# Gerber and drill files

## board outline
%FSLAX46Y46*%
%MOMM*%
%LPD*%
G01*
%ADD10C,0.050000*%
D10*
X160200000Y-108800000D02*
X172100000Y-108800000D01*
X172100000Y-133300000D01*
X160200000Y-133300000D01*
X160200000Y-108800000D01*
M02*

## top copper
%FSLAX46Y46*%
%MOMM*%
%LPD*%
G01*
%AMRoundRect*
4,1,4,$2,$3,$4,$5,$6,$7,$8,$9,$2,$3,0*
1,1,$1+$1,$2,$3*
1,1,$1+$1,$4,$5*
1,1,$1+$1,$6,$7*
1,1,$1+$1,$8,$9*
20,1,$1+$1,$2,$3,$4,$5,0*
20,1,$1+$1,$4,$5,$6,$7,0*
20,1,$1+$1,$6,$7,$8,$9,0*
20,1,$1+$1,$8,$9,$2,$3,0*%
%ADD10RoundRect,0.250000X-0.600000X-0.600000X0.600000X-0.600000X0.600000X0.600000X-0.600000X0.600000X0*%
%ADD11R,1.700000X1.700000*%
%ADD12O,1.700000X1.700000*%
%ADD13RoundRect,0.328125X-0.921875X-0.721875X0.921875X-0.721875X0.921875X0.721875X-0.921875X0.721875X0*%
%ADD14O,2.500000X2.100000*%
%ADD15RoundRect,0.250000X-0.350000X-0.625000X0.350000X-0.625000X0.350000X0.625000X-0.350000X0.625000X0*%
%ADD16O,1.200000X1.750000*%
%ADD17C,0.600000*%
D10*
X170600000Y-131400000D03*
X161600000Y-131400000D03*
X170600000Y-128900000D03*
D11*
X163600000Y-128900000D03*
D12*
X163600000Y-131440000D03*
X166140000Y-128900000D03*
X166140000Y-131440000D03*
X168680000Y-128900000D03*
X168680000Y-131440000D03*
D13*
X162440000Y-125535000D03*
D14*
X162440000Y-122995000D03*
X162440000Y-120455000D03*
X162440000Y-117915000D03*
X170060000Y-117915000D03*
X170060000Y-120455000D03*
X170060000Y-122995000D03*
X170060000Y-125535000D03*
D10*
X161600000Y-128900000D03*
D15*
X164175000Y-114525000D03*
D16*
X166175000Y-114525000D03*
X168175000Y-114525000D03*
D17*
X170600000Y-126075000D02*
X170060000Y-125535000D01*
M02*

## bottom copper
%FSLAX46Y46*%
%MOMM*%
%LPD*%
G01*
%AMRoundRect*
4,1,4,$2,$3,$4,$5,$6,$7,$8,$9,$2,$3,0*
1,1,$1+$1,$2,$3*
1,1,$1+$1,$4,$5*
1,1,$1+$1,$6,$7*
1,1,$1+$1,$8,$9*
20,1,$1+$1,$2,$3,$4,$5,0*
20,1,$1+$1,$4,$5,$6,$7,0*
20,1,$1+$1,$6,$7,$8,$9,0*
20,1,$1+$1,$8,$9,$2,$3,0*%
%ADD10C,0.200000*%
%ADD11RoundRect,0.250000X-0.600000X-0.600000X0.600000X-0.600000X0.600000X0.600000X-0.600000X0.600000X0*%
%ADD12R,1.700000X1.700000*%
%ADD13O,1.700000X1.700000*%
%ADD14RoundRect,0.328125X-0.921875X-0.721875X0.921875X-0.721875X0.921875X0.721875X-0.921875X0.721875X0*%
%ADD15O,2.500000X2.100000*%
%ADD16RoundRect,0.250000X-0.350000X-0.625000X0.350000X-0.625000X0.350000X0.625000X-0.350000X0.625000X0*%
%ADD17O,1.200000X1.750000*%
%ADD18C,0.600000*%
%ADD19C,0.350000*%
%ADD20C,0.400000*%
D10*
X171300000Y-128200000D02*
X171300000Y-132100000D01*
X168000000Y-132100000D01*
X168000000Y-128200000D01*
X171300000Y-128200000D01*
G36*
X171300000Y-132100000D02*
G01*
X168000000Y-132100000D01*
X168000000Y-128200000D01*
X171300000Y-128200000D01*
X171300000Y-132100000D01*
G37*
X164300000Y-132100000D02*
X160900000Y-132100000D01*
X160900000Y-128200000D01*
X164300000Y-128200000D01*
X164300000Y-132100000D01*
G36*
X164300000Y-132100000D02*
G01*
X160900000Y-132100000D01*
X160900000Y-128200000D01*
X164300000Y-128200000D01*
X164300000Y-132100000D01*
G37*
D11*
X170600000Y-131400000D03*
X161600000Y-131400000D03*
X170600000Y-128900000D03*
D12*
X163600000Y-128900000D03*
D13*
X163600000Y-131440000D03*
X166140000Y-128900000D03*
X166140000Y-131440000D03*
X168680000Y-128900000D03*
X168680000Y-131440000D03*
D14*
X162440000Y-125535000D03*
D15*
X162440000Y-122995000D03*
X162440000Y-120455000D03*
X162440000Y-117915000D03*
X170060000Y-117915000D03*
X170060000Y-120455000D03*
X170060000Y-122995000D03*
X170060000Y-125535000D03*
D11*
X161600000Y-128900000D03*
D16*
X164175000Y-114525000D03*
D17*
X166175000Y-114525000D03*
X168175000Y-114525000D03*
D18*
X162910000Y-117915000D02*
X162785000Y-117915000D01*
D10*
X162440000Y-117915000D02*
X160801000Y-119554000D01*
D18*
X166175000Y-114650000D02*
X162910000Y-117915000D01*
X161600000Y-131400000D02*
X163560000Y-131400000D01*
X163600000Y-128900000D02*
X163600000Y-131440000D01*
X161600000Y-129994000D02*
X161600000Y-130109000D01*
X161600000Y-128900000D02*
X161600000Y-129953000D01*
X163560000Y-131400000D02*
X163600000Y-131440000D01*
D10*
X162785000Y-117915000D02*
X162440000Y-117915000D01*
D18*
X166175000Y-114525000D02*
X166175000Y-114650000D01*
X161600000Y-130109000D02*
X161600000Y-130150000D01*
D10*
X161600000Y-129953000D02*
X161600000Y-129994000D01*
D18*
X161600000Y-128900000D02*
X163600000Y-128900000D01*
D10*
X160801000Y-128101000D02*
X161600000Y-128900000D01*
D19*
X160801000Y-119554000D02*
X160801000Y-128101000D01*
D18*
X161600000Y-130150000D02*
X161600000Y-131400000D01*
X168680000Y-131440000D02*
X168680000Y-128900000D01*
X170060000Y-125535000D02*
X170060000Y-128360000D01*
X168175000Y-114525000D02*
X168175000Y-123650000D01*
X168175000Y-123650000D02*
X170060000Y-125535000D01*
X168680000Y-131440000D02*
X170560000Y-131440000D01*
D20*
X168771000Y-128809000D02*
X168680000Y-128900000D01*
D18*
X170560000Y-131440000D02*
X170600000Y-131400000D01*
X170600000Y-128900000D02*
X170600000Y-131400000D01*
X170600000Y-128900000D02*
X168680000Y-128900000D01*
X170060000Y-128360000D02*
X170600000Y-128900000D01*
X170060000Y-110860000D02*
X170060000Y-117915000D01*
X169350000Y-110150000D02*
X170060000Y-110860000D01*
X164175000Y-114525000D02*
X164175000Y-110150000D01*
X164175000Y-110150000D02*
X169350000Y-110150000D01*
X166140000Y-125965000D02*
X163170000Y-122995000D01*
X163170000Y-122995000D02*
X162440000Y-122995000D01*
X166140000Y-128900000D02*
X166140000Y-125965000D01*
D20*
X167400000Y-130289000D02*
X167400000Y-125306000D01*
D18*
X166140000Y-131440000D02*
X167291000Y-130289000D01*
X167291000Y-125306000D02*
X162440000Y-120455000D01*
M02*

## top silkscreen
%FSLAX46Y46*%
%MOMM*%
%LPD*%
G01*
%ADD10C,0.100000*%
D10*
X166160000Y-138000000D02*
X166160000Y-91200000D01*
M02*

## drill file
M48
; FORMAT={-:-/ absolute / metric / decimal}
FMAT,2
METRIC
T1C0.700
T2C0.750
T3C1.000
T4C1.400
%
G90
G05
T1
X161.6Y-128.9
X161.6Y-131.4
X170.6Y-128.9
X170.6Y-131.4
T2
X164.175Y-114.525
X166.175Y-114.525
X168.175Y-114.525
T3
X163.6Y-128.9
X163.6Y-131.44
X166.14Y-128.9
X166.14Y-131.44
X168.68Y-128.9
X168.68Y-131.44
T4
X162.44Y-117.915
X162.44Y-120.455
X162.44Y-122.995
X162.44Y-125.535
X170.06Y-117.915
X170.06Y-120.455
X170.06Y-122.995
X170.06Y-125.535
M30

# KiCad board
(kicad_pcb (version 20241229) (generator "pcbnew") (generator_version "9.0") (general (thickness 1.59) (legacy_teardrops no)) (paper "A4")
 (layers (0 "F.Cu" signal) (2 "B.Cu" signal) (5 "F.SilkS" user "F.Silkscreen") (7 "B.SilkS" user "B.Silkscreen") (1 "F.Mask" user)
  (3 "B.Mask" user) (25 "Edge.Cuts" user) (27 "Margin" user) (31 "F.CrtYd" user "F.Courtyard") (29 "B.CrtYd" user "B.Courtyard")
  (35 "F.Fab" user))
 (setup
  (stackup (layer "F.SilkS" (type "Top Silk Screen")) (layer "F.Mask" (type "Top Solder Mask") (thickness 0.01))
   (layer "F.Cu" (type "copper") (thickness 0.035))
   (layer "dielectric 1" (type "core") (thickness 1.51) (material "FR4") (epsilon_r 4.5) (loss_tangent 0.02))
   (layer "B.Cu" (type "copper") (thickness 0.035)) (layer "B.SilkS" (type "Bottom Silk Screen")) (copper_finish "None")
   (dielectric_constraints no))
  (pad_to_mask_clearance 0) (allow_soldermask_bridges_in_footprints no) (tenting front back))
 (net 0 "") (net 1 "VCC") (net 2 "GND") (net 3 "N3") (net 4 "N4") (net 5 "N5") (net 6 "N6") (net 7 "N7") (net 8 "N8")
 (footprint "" (layer "F.Cu") (at 170.6 131.4)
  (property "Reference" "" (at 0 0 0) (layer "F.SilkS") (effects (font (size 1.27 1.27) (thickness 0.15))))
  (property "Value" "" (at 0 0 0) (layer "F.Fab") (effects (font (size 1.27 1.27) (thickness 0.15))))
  (pad "1" thru_hole roundrect (at 0 0) (size 1.7 1.7) (drill 0.7) (layers "*.Cu" "*.Mask") (remove_unused_layers no)
   (roundrect_rratio 0.147059) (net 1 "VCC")))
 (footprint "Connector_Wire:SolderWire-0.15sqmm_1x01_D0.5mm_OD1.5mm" (layer "B.Cu") (at 161.6 131.4)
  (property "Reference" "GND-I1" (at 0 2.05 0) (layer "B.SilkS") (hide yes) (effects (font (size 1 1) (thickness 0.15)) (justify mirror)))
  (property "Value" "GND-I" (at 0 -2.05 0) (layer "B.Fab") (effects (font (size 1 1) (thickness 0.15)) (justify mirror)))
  (pad "1" thru_hole roundrect (at 0 0) (size 1.7 1.7) (drill 0.7) (layers "*.Cu" "*.Mask") (remove_unused_layers no)
   (roundrect_rratio 0.147059) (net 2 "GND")))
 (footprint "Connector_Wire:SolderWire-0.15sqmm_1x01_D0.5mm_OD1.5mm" (layer "B.Cu") (at 170.6 128.9)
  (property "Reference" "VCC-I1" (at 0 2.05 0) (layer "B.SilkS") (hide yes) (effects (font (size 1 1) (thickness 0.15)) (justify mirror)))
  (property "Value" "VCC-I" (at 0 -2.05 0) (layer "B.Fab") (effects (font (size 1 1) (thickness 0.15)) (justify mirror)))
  (pad "1" thru_hole roundrect (at 0 0) (size 1.7 1.7) (drill 0.7) (layers "*.Cu" "*.Mask") (remove_unused_layers no)
   (roundrect_rratio 0.147059) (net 1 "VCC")))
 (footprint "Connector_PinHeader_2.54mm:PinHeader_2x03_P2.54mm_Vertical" (layer "B.Cu") (at 163.6 128.9 -90)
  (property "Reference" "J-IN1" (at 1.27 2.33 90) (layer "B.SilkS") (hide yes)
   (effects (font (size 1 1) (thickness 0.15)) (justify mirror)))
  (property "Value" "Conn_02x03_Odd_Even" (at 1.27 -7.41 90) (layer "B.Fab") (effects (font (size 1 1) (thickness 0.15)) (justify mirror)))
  (pad "1" thru_hole rect (at 0 0 270) (size 1.7 1.7) (drill 1) (layers "*.Cu" "*.Mask") (remove_unused_layers no) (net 2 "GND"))
  (pad "2" thru_hole oval (at 2.54 0 270) (size 1.7 1.7) (drill 1) (layers "*.Cu" "*.Mask") (remove_unused_layers no) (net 2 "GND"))
  (pad "3" thru_hole oval (at 0 -2.54 270) (size 1.7 1.7) (drill 1) (layers "*.Cu" "*.Mask") (remove_unused_layers no) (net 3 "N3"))
  (pad "4" thru_hole oval (at 2.54 -2.54 270) (size 1.7 1.7) (drill 1) (layers "*.Cu" "*.Mask") (remove_unused_layers no) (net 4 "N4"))
  (pad "5" thru_hole oval (at 0 -5.08 270) (size 1.7 1.7) (drill 1) (layers "*.Cu" "*.Mask") (remove_unused_layers no) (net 1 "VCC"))
  (pad "6" thru_hole oval (at 2.54 -5.08 270) (size 1.7 1.7) (drill 1) (layers "*.Cu" "*.Mask") (remove_unused_layers no) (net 1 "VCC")))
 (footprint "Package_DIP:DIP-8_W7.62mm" (layer "B.Cu") (at 162.44 125.535)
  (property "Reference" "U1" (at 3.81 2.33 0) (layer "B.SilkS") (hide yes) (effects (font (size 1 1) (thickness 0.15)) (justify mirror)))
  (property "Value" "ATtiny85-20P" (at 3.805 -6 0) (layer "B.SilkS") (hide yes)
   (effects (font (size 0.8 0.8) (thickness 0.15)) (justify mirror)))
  (pad "1" thru_hole roundrect (at 0 0) (size 2.5 2.1) (drill 1.4) (layers "*.Cu" "*.Mask") (remove_unused_layers no)
   (roundrect_rratio 0.15625) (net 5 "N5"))
  (pad "2" thru_hole oval (at 0 -2.54) (size 2.5 2.1) (drill 1.4) (layers "*.Cu" "*.Mask") (remove_unused_layers no) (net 3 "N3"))
  (pad "3" thru_hole oval (at 0 -5.08) (size 2.5 2.1) (drill 1.4) (layers "*.Cu" "*.Mask") (remove_unused_layers no) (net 4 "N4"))
  (pad "4" thru_hole oval (at 0 -7.62) (size 2.5 2.1) (drill 1.4) (layers "*.Cu" "*.Mask") (remove_unused_layers no) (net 2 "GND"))
  (pad "5" thru_hole oval (at 7.62 -7.62) (size 2.5 2.1) (drill 1.4) (layers "*.Cu" "*.Mask") (remove_unused_layers no) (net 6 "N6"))
  (pad "6" thru_hole oval (at 7.62 -5.08) (size 2.5 2.1) (drill 1.4) (layers "*.Cu" "*.Mask") (remove_unused_layers no) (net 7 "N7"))
  (pad "7" thru_hole oval (at 7.62 -2.54) (size 2.5 2.1) (drill 1.4) (layers "*.Cu" "*.Mask") (remove_unused_layers no) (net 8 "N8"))
  (pad "8" thru_hole oval (at 7.62 0) (size 2.5 2.1) (drill 1.4) (layers "*.Cu" "*.Mask") (remove_unused_layers no) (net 1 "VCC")))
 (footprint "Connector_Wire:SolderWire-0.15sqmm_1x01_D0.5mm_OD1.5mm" (layer "B.Cu") (at 161.6 128.9)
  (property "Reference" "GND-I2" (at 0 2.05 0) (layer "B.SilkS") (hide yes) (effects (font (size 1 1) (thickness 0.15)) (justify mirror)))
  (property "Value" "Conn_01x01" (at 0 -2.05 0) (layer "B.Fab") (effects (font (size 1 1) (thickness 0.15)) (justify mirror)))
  (pad "1" thru_hole roundrect (at 0 0) (size 1.7 1.7) (drill 0.7) (layers "*.Cu" "*.Mask") (remove_unused_layers no)
   (roundrect_rratio 0.147059) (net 2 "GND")))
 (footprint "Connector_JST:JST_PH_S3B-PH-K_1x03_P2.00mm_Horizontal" (layer "B.Cu") (at 164.175 114.525)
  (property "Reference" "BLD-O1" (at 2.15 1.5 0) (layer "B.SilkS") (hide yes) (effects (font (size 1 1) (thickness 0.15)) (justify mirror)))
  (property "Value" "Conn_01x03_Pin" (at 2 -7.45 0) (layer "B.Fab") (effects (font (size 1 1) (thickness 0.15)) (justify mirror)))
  (pad "1" thru_hole roundrect (at 0 0) (size 1.2 1.75) (drill 0.75) (layers "*.Cu" "*.Mask") (remove_unused_layers no)
   (roundrect_rratio 0.208333) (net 6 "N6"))
  (pad "2" thru_hole oval (at 2 0) (size 1.2 1.75) (drill 0.75) (layers "*.Cu" "*.Mask") (remove_unused_layers no) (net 2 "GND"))
  (pad "3" thru_hole oval (at 4 0) (size 1.2 1.75) (drill 0.75) (layers "*.Cu" "*.Mask") (remove_unused_layers no) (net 1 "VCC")))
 (gr_poly
  (pts (xy 171.3 128.2) (xy 171.3 132.1) (xy 168 132.1) (xy 168 128.2)) (stroke (width 0.2) (type solid)) (fill yes) (layer "B.Cu") (net 1))
 (gr_poly
  (pts (xy 164.3 132.1) (xy 160.9 132.1) (xy 160.9 128.2) (xy 164.3 128.2)) (stroke (width 0.2) (type solid)) (fill yes) (layer "B.Cu")
  (net 2))
 (gr_line (start 166.16 138) (end 166.16 91.2) (stroke (width 0.1) (type default)) (layer "F.SilkS"))
 (gr_rect (start 160.2 108.8) (end 172.1 133.3) (stroke (width 0.05) (type default)) (fill no) (layer "Edge.Cuts"))
 (segment (start 162.91 117.915) (end 162.785 117.915) (width 0.6) (layer "B.Cu") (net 2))
 (segment (start 162.44 117.915) (end 160.801 119.554) (width 0.2) (layer "B.Cu") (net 2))
 (segment (start 166.175 114.65) (end 162.91 117.915) (width 0.6) (layer "B.Cu") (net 2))
 (segment (start 161.6 131.4) (end 163.56 131.4) (width 0.6) (layer "B.Cu") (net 2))
 (segment (start 163.6 128.9) (end 163.6 131.44) (width 0.6) (layer "B.Cu") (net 2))
 (segment (start 161.6 129.994) (end 161.6 130.109) (width 0.6) (layer "B.Cu") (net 2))
 (segment (start 161.6 128.9) (end 161.6 129.953) (width 0.6) (layer "B.Cu") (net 2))
 (segment (start 163.56 131.4) (end 163.6 131.44) (width 0.6) (layer "B.Cu") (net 2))
 (segment (start 162.785 117.915) (end 162.44 117.915) (width 0.2) (layer "B.Cu") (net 2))
 (segment (start 166.175 114.525) (end 166.175 114.65) (width 0.6) (layer "B.Cu") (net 2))
 (segment (start 161.6 130.109) (end 161.6 130.15) (width 0.6) (layer "B.Cu") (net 2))
 (segment (start 161.6 129.953) (end 161.6 129.994) (width 0.2) (layer "B.Cu") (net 2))
 (segment (start 161.6 128.9) (end 163.6 128.9) (width 0.6) (layer "B.Cu") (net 2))
 (segment (start 160.801 128.101) (end 161.6 128.9) (width 0.2) (layer "B.Cu") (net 2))
 (segment (start 160.801 119.554) (end 160.801 128.101) (width 0.35) (layer "B.Cu") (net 2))
 (segment (start 161.6 130.15) (end 161.6 131.4) (width 0.6) (layer "B.Cu") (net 2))
 (segment (start 170.6 126.075) (end 170.06 125.535) (width 0.6) (layer "F.Cu") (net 1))
 (segment (start 168.68 131.44) (end 168.68 128.9) (width 0.6) (layer "B.Cu") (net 1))
 (segment (start 170.06 125.535) (end 170.06 128.36) (width 0.6) (layer "B.Cu") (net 1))
 (segment (start 168.175 114.525) (end 168.175 123.65) (width 0.6) (layer "B.Cu") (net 1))
 (segment (start 168.175 123.65) (end 170.06 125.535) (width 0.6) (layer "B.Cu") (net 1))
 (segment (start 168.68 131.44) (end 170.56 131.44) (width 0.6) (layer "B.Cu") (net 1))
 (segment (start 168.771 128.809) (end 168.68 128.9) (width 0.4) (layer "B.Cu") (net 1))
 (segment (start 170.56 131.44) (end 170.6 131.4) (width 0.6) (layer "B.Cu") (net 1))
 (segment (start 170.6 128.9) (end 170.6 131.4) (width 0.6) (layer "B.Cu") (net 1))
 (segment (start 170.6 128.9) (end 168.68 128.9) (width 0.6) (layer "B.Cu") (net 1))
 (segment (start 170.06 128.36) (end 170.6 128.9) (width 0.6) (layer "B.Cu") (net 1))
 (segment (start 170.06 110.86) (end 170.06 117.915) (width 0.6) (layer "B.Cu") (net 6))
 (segment (start 169.35 110.15) (end 170.06 110.86) (width 0.6) (layer "B.Cu") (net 6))
 (segment (start 164.175 114.525) (end 164.175 110.15) (width 0.6) (layer "B.Cu") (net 6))
 (segment (start 164.175 110.15) (end 169.35 110.15) (width 0.6) (layer "B.Cu") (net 6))
 (segment (start 166.14 125.965) (end 163.17 122.995) (width 0.6) (layer "B.Cu") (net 3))
 (segment (start 163.17 122.995) (end 162.44 122.995) (width 0.6) (layer "B.Cu") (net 3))
 (segment (start 166.14 128.9) (end 166.14 125.965) (width 0.6) (layer "B.Cu") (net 3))
 (segment (start 167.4 130.289) (end 167.4 125.306) (width 0.4) (layer "B.Cu") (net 4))
 (segment (start 166.14 131.44) (end 167.291 130.289) (width 0.6) (layer "B.Cu") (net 4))
 (segment (start 167.291 125.306) (end 162.44 120.455) (width 0.6) (layer "B.Cu") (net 4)))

